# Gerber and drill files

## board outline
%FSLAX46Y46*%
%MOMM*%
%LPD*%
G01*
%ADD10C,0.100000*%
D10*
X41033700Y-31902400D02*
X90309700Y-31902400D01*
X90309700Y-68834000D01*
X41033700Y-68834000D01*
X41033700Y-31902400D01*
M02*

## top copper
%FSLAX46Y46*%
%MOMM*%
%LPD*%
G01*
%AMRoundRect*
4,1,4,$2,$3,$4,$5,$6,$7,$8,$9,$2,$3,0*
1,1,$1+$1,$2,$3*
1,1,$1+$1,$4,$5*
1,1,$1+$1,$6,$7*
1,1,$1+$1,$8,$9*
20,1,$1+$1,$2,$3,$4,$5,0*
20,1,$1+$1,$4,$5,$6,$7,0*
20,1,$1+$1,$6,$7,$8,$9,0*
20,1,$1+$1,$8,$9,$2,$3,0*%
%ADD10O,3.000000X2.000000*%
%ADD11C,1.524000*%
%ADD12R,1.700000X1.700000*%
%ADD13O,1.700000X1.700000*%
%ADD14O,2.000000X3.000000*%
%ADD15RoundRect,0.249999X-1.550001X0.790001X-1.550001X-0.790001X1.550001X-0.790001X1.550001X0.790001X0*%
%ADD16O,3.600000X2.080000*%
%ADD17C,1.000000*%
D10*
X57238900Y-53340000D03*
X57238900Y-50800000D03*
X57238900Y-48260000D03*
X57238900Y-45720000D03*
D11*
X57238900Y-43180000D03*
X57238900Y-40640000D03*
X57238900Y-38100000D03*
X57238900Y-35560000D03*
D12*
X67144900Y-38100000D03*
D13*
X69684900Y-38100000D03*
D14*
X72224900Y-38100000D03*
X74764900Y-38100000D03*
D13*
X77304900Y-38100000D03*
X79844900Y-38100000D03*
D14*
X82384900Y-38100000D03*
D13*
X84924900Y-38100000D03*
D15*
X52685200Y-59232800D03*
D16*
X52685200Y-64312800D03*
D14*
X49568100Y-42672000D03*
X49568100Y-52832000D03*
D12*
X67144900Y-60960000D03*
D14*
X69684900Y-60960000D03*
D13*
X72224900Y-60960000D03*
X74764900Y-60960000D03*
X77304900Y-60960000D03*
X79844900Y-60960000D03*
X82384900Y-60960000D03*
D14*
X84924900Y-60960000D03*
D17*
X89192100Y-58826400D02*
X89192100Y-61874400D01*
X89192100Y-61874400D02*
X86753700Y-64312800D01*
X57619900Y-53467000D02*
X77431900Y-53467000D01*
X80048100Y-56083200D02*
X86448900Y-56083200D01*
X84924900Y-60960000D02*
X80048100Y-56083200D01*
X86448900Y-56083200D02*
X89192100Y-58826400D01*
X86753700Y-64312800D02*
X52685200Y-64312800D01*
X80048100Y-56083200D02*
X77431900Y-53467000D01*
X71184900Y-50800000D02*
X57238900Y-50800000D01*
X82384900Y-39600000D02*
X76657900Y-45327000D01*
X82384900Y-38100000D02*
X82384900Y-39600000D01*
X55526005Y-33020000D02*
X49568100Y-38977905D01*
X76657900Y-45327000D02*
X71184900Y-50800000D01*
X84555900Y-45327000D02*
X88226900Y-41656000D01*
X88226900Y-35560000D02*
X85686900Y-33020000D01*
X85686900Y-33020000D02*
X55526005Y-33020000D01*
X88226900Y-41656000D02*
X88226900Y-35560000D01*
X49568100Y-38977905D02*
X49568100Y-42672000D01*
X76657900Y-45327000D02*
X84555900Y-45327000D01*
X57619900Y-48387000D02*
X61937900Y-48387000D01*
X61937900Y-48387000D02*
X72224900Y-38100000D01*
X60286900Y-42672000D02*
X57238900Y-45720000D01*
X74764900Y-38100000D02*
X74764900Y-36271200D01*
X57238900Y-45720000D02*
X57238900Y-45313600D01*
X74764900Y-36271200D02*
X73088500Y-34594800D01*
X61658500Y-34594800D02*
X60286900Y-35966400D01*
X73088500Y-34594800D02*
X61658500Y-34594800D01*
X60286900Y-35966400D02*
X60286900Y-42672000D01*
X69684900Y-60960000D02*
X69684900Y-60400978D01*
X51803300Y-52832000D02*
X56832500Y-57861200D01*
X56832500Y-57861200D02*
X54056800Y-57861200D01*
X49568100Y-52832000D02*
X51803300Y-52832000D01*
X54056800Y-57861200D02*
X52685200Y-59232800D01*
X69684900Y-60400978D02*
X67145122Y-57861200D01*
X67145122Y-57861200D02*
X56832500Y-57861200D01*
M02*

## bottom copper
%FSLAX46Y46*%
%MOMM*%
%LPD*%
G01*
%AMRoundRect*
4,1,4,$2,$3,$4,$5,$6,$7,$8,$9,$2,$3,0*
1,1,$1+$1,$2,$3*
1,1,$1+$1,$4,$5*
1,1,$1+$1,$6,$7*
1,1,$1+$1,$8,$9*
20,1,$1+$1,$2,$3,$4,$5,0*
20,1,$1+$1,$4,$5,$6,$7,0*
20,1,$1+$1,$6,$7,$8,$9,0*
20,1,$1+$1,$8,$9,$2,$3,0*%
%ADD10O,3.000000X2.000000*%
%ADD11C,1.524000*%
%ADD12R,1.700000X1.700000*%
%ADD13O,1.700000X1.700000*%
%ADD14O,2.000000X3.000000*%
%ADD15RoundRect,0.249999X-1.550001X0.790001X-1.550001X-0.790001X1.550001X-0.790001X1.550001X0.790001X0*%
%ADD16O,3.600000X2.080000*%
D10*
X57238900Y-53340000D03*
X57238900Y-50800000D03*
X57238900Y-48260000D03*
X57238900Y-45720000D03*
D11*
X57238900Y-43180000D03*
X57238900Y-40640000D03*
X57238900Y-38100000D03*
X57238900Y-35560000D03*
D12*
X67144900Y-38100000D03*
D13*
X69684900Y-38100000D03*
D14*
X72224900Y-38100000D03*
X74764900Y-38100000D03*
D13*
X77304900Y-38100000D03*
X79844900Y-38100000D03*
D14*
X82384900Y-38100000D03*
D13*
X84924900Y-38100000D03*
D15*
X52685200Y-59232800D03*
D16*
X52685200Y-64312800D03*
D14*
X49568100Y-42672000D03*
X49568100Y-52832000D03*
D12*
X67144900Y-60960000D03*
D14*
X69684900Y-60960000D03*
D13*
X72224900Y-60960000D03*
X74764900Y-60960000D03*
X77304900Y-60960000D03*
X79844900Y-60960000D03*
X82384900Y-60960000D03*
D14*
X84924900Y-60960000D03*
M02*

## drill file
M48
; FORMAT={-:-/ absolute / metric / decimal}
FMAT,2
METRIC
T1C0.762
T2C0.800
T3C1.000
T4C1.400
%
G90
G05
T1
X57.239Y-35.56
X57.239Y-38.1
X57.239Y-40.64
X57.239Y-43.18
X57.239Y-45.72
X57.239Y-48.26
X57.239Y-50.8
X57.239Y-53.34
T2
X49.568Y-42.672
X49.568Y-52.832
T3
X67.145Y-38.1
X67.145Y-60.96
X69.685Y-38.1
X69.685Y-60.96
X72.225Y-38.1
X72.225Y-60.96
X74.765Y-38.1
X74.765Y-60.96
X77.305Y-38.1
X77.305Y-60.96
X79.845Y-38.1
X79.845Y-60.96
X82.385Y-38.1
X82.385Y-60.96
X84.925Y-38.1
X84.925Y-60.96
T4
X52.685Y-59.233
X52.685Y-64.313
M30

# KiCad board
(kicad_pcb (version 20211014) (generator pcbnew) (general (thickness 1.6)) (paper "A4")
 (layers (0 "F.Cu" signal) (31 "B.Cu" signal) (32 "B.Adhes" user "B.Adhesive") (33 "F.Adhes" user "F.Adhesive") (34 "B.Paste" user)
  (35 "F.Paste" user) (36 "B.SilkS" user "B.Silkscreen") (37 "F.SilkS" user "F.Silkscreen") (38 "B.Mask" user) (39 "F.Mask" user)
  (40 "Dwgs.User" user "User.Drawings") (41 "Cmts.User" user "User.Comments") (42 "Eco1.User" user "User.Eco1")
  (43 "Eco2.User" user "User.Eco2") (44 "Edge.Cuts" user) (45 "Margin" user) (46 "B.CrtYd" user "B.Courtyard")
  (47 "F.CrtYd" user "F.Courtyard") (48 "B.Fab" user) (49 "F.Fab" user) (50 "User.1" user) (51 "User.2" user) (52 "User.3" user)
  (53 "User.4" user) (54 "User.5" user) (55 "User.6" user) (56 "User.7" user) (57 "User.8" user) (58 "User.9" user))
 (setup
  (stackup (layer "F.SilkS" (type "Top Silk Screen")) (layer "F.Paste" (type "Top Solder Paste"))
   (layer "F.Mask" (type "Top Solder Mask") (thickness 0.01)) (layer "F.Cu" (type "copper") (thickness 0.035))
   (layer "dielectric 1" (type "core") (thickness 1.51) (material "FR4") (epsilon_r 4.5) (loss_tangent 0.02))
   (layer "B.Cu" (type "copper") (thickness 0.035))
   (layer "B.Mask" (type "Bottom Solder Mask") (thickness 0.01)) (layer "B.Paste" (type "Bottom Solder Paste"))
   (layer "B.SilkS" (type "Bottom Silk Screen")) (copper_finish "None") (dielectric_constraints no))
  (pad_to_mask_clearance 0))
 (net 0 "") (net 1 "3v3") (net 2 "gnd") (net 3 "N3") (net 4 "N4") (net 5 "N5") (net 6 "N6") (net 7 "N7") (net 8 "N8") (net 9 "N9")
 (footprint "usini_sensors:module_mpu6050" (layer "F.Cu") (at 57.2389 35.56 180)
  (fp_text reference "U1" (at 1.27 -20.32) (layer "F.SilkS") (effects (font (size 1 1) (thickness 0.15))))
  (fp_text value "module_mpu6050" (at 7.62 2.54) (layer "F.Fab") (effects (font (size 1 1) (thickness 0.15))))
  (pad "1" thru_hole oval locked (at 0 -17.78 180) (size 3 2) (drill 0.762) (layers *.Cu *.Mask) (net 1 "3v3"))
  (pad "2" thru_hole oval locked (at 0 -15.24 180) (size 3 2) (drill 0.762) (layers *.Cu *.Mask) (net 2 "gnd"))
  (pad "3" thru_hole oval locked (at 0 -12.7 180) (size 3 2) (drill 0.762) (layers *.Cu *.Mask) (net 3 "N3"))
  (pad "4" thru_hole oval locked (at 0 -10.16 180) (size 3 2) (drill 0.762) (layers *.Cu *.Mask) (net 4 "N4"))
  (pad "5" thru_hole circle locked (at 0 -7.62 180) (size 1.524 1.524) (drill 0.762) (layers *.Cu *.Mask) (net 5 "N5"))
  (pad "6" thru_hole circle locked (at 0 -5.08 180) (size 1.524 1.524) (drill 0.762) (layers *.Cu *.Mask) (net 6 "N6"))
  (pad "7" thru_hole circle locked (at 0 -2.54 180) (size 1.524 1.524) (drill 0.762) (layers *.Cu *.Mask) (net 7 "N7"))
  (pad "8" thru_hole circle locked (at 0 0 180) (size 1.524 1.524) (drill 0.762) (layers *.Cu *.Mask) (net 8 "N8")))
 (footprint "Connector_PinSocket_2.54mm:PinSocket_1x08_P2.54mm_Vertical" (layer "F.Cu") (at 67.1449 38.1 90)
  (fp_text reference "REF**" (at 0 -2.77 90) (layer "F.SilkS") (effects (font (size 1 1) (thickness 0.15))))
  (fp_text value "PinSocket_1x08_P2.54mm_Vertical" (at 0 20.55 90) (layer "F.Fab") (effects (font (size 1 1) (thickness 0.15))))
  (pad "1" thru_hole rect (at 0 0 90) (size 1.7 1.7) (drill 1) (layers *.Cu *.Mask))
  (pad "2" thru_hole oval (at 0 2.54 90) (size 1.7 1.7) (drill 1) (layers *.Cu *.Mask))
  (pad "3" thru_hole oval (at 0 5.08 90) (size 3 2) (drill 1) (layers *.Cu *.Mask))
  (pad "4" thru_hole oval (at 0 7.62 90) (size 3 2) (drill 1) (layers *.Cu *.Mask) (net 4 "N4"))
  (pad "5" thru_hole oval (at 0 10.16 90) (size 1.7 1.7) (drill 1) (layers *.Cu *.Mask))
  (pad "6" thru_hole oval (at 0 12.7 90) (size 1.7 1.7) (drill 1) (layers *.Cu *.Mask))
  (pad "7" thru_hole oval (at 0 15.24 90) (size 3 2) (drill 1) (layers *.Cu *.Mask) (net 2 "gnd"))
  (pad "8" thru_hole oval (at 0 17.78 90) (size 1.7 1.7) (drill 1) (layers *.Cu *.Mask)))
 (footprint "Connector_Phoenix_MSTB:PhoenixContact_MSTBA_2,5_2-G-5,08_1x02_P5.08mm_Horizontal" (layer "F.Cu") (at 52.6852 59.2328 -90)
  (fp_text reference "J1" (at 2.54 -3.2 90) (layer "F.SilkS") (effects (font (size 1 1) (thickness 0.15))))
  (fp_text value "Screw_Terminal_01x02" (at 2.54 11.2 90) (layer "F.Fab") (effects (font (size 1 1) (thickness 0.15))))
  (pad "1" thru_hole roundrect (at 0 0 270) (size 2.08 3.6) (drill 1.4) (layers *.Cu *.Mask) (roundrect_rratio 0.120192) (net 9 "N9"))
  (pad "2" thru_hole oval (at 5.08 0 270) (size 2.08 3.6) (drill 1.4) (layers *.Cu *.Mask) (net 1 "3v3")))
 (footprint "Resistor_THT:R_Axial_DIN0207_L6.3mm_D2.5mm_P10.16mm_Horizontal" (layer "F.Cu") (at 49.5681 42.672 -90)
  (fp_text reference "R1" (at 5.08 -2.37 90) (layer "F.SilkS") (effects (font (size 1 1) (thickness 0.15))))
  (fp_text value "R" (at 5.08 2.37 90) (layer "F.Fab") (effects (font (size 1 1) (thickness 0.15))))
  (pad "1" thru_hole oval (at 0 0 270) (size 3 2) (drill 0.8) (layers *.Cu *.Mask) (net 2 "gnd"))
  (pad "2" thru_hole oval (at 10.16 0 270) (size 3 2) (drill 0.8) (layers *.Cu *.Mask) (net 9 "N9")))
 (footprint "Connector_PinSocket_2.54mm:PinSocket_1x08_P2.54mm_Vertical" (layer "F.Cu") (at 67.1449 60.96 90)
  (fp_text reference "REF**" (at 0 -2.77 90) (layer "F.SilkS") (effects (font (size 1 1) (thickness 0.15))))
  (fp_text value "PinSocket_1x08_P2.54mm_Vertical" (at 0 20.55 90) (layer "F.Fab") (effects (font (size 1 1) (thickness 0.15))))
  (pad "1" thru_hole rect (at 0 0 90) (size 1.7 1.7) (drill 1) (layers *.Cu *.Mask))
  (pad "2" thru_hole oval (at 0 2.54 90) (size 3 2) (drill 1) (layers *.Cu *.Mask) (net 9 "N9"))
  (pad "3" thru_hole oval (at 0 5.08 90) (size 1.7 1.7) (drill 1) (layers *.Cu *.Mask))
  (pad "4" thru_hole oval (at 0 7.62 90) (size 1.7 1.7) (drill 1) (layers *.Cu *.Mask))
  (pad "5" thru_hole oval (at 0 10.16 90) (size 1.7 1.7) (drill 1) (layers *.Cu *.Mask))
  (pad "6" thru_hole oval (at 0 12.7 90) (size 1.7 1.7) (drill 1) (layers *.Cu *.Mask))
  (pad "7" thru_hole oval (at 0 15.24 90) (size 1.7 1.7) (drill 1) (layers *.Cu *.Mask))
  (pad "8" thru_hole oval (at 0 17.78 90) (size 3 2) (drill 1) (layers *.Cu *.Mask) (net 1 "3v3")))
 (gr_rect (start 41.0337 68.834) (end 90.3097 31.9024) (layer "Edge.Cuts") (width 0.1) (fill none))
 (segment (start 89.1921 58.8264) (end 89.1921 61.8744) (width 1) (layer "F.Cu") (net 1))
 (segment (start 89.1921 61.8744) (end 86.7537 64.3128) (width 1) (layer "F.Cu") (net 1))
 (segment (start 57.6199 53.467) (end 77.4319 53.467) (width 1) (layer "F.Cu") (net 1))
 (segment (start 80.0481 56.0832) (end 86.4489 56.0832) (width 1) (layer "F.Cu") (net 1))
 (segment (start 84.9249 60.96) (end 80.0481 56.0832) (width 1) (layer "F.Cu") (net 1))
 (segment (start 86.4489 56.0832) (end 89.1921 58.8264) (width 1) (layer "F.Cu") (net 1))
 (segment (start 86.7537 64.3128) (end 52.6852 64.3128) (width 1) (layer "F.Cu") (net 1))
 (segment (start 80.0481 56.0832) (end 77.4319 53.467) (width 1) (layer "F.Cu") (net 1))
 (segment (start 71.1849 50.8) (end 57.2389 50.8) (width 1) (layer "F.Cu") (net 2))
 (segment (start 82.3849 39.6) (end 76.6579 45.327) (width 1) (layer "F.Cu") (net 2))
 (segment (start 82.3849 38.1) (end 82.3849 39.6) (width 1) (layer "F.Cu") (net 2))
 (segment (start 55.526005 33.02) (end 49.5681 38.977905) (width 1) (layer "F.Cu") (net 2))
 (segment (start 76.6579 45.327) (end 71.1849 50.8) (width 1) (layer "F.Cu") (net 2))
 (segment (start 84.5559 45.327) (end 88.2269 41.656) (width 1) (layer "F.Cu") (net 2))
 (segment (start 88.2269 35.56) (end 85.6869 33.02) (width 1) (layer "F.Cu") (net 2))
 (segment (start 85.6869 33.02) (end 55.526005 33.02) (width 1) (layer "F.Cu") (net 2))
 (segment (start 88.2269 41.656) (end 88.2269 35.56) (width 1) (layer "F.Cu") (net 2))
 (segment (start 49.5681 38.977905) (end 49.5681 42.672) (width 1) (layer "F.Cu") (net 2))
 (segment (start 76.6579 45.327) (end 84.5559 45.327) (width 1) (layer "F.Cu") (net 2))
 (segment (start 57.6199 48.387) (end 61.9379 48.387) (width 1) (layer "F.Cu") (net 3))
 (segment (start 61.9379 48.387) (end 72.2249 38.1) (width 1) (layer "F.Cu") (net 3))
 (segment (start 60.2869 42.672) (end 57.2389 45.72) (width 1) (layer "F.Cu") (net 4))
 (segment (start 74.7649 38.1) (end 74.7649 36.2712) (width 1) (layer "F.Cu") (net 4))
 (segment (start 57.2389 45.72) (end 57.2389 45.3136) (width 1) (layer "F.Cu") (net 4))
 (segment (start 74.7649 36.2712) (end 73.0885 34.5948) (width 1) (layer "F.Cu") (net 4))
 (segment (start 61.6585 34.5948) (end 60.2869 35.9664) (width 1) (layer "F.Cu") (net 4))
 (segment (start 73.0885 34.5948) (end 61.6585 34.5948) (width 1) (layer "F.Cu") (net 4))
 (segment (start 60.2869 35.9664) (end 60.2869 42.672) (width 1) (layer "F.Cu") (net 4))
 (segment (start 69.6849 60.96) (end 69.6849 60.400978) (width 1) (layer "F.Cu") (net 9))
 (segment (start 51.8033 52.832) (end 56.8325 57.8612) (width 1) (layer "F.Cu") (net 9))
 (segment (start 56.8325 57.8612) (end 54.0568 57.8612) (width 1) (layer "F.Cu") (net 9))
 (segment (start 49.5681 52.832) (end 51.8033 52.832) (width 1) (layer "F.Cu") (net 9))
 (segment (start 54.0568 57.8612) (end 52.6852 59.2328) (width 1) (layer "F.Cu") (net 9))
 (segment (start 69.6849 60.400978) (end 67.145122 57.8612) (width 1) (layer "F.Cu") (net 9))
 (segment (start 67.145122 57.8612) (end 56.8325 57.8612) (width 1) (layer "F.Cu") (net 9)))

